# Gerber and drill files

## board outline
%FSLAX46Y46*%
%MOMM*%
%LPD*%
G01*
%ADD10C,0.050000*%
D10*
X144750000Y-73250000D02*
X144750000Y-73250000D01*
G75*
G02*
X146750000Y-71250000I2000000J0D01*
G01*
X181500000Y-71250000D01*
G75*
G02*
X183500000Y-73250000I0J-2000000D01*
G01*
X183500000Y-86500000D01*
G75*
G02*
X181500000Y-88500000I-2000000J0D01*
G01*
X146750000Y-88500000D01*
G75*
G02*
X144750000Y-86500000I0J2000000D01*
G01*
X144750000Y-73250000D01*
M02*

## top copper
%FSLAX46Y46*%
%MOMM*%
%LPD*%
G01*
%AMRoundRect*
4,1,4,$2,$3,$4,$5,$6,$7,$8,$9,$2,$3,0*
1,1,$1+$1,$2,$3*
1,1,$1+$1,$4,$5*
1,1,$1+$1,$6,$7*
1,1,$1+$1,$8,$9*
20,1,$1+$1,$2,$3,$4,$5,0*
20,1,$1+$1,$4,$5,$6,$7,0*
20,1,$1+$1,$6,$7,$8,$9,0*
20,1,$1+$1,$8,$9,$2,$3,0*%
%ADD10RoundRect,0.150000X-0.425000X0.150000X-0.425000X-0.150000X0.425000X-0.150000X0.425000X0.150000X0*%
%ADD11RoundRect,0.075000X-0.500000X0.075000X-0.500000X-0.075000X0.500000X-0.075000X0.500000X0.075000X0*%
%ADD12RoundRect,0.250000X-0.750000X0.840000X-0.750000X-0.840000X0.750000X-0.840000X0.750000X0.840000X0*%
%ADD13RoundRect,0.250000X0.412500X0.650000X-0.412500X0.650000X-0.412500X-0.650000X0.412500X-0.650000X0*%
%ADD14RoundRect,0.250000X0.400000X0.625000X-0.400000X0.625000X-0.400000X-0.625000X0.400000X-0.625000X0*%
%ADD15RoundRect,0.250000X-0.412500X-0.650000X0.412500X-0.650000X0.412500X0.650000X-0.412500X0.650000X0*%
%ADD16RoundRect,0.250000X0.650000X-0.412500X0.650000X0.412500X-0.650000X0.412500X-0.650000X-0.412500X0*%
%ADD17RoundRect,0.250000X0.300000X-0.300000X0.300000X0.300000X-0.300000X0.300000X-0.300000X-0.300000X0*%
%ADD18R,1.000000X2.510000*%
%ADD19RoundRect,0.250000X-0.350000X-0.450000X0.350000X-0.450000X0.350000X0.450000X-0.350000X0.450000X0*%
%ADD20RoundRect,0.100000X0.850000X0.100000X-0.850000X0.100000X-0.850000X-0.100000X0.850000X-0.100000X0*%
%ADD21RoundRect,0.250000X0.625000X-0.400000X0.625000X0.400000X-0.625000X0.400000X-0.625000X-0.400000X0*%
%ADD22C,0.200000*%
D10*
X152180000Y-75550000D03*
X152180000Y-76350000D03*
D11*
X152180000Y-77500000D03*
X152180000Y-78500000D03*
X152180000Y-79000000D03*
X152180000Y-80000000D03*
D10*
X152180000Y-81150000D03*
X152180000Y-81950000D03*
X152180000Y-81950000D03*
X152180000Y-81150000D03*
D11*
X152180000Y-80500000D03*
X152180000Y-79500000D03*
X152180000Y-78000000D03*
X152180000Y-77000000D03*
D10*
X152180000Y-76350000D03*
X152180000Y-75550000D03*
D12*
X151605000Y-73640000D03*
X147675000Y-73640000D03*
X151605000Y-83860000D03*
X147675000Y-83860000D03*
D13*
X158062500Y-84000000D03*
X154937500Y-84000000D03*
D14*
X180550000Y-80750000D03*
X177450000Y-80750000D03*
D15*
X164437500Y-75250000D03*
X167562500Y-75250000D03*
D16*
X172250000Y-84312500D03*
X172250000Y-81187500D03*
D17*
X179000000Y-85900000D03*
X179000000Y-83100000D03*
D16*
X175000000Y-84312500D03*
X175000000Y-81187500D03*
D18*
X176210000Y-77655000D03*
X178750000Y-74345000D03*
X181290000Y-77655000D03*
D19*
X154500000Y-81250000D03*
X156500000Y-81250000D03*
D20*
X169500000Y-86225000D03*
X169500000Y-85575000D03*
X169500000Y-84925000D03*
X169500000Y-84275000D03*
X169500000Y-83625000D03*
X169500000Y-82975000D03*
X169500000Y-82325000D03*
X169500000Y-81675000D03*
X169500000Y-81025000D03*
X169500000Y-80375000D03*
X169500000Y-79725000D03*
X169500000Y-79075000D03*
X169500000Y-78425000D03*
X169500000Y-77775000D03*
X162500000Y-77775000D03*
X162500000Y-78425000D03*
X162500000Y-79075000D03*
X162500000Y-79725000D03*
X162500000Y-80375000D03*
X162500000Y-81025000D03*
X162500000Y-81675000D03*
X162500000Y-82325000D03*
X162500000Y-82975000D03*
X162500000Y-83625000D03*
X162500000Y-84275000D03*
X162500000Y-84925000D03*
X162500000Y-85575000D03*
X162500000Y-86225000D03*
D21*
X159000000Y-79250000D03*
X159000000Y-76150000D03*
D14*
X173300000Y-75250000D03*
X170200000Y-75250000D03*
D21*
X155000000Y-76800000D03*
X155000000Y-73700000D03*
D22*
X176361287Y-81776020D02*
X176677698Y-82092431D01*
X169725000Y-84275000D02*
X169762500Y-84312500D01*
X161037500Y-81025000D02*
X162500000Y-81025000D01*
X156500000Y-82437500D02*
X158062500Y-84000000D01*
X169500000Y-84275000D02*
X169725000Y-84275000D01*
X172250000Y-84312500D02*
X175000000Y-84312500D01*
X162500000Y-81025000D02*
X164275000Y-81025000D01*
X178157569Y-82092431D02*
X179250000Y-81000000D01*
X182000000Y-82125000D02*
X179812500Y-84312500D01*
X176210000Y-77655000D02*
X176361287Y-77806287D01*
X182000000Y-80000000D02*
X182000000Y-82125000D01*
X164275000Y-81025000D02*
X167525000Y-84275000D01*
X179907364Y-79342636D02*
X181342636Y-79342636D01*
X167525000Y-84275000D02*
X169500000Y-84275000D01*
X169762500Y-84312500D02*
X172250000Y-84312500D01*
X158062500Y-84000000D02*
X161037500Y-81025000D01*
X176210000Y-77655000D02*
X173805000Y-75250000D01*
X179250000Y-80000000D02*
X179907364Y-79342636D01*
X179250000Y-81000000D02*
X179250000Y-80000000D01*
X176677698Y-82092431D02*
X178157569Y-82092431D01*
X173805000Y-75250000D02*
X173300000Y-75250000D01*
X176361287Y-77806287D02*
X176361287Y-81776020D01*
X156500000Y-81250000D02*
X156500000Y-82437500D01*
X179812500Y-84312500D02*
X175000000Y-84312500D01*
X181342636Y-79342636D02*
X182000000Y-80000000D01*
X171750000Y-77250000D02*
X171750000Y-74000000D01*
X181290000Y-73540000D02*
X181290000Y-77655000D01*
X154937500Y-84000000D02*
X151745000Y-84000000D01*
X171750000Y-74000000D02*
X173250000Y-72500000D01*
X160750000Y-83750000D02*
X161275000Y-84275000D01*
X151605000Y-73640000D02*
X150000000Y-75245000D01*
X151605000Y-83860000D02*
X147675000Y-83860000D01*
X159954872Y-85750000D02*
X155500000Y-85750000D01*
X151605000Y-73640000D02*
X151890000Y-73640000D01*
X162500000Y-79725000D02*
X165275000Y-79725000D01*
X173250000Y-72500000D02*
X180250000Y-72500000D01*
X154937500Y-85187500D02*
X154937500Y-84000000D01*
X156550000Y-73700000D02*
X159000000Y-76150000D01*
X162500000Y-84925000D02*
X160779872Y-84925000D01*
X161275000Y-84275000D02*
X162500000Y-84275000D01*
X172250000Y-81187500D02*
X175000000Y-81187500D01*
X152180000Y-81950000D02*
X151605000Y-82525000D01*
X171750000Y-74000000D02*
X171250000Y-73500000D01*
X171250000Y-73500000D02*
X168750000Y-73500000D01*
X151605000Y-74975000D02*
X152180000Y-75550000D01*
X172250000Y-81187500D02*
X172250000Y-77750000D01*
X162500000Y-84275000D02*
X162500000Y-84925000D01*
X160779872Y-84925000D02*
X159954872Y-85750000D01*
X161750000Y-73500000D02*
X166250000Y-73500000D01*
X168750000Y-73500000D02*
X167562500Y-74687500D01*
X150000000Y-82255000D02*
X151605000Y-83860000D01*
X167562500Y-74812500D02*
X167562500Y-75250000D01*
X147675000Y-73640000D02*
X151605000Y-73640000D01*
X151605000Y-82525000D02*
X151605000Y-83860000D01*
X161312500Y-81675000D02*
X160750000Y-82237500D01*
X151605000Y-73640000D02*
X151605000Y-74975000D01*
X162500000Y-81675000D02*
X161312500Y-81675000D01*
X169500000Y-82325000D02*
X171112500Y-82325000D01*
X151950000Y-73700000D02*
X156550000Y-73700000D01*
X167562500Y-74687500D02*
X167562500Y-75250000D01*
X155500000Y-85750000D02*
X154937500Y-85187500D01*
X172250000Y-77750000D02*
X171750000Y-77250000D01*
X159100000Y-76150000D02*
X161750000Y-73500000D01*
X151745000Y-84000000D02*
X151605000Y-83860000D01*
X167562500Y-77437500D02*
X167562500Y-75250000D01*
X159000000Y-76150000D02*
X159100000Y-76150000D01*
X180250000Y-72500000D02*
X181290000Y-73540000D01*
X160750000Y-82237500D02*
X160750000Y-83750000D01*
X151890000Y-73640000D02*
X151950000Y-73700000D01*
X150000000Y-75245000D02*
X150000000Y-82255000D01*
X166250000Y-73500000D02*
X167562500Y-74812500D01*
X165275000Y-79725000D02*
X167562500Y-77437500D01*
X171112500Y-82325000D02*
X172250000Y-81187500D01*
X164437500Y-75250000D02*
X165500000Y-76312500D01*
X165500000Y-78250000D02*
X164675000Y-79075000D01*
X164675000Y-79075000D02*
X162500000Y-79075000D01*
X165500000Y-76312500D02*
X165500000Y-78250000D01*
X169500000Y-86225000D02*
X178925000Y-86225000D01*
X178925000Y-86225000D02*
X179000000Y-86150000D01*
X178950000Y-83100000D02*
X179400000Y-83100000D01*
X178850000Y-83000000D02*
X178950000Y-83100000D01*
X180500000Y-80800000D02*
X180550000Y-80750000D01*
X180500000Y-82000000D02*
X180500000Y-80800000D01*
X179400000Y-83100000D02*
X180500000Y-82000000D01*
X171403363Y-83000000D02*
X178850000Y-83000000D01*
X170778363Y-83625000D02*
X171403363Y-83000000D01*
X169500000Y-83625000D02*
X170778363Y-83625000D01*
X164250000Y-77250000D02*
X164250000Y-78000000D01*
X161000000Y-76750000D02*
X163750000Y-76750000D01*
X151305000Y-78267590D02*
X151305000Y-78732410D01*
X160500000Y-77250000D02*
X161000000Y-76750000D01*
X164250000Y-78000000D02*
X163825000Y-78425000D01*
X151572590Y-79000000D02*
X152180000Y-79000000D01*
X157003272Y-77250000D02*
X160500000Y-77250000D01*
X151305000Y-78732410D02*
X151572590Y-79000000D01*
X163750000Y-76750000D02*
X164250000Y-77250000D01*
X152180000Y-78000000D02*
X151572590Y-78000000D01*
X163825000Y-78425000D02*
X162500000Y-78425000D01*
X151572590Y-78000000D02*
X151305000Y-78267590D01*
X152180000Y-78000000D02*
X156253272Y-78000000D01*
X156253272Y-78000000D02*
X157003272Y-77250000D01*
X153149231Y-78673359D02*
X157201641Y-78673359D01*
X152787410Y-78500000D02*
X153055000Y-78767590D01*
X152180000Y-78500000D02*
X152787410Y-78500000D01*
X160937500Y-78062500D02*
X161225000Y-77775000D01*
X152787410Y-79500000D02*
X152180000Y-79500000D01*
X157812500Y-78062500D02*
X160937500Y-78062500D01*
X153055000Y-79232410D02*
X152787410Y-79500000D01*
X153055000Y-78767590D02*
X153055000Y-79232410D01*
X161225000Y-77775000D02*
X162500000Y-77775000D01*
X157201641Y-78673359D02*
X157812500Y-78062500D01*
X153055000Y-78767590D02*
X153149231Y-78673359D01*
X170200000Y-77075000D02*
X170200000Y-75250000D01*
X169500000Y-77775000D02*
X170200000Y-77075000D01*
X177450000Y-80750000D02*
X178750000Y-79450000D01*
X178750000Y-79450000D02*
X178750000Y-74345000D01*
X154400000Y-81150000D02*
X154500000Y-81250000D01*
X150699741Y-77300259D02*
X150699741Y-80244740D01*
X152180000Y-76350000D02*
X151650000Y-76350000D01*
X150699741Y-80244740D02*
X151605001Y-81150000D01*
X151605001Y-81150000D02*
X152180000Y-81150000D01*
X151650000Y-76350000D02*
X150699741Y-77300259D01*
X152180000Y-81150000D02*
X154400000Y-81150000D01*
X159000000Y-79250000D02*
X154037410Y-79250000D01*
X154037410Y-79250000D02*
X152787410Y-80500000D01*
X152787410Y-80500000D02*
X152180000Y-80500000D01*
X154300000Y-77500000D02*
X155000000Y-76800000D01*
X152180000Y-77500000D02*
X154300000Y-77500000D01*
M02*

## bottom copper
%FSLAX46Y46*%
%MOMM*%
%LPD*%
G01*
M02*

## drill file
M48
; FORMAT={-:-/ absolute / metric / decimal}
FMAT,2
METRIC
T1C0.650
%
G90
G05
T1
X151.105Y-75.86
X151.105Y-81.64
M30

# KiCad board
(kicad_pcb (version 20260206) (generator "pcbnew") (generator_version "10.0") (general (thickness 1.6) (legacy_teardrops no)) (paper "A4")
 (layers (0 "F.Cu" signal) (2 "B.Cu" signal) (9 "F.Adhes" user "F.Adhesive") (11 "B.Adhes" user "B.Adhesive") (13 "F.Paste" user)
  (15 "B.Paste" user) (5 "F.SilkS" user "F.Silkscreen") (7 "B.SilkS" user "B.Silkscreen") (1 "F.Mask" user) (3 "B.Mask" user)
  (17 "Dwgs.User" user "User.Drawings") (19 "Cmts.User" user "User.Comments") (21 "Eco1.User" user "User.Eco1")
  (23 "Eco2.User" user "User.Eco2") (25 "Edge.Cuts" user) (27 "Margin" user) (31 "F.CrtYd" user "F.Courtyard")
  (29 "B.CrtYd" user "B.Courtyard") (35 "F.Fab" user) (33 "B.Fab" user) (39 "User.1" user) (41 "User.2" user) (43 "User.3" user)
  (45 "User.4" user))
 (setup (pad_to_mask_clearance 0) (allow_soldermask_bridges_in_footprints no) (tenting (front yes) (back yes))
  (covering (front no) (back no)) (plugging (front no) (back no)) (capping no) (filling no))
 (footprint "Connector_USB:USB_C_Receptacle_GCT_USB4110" (layer "F.Cu") (at 148.5 78.75 -90)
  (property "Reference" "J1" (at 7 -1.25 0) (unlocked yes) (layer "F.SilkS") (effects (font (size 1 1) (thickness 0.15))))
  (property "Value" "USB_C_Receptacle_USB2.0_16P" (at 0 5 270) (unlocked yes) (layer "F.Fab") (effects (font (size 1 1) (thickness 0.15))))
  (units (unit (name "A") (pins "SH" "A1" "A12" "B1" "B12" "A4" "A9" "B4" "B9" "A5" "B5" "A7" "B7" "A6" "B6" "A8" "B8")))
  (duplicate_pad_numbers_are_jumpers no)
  (pad "" np_thru_hole circle (at -2.89 -2.605 270) (size 0.65 0.65) (drill 0.65) (layers "*.Cu" "*.Mask"))
  (pad "" np_thru_hole circle (at 2.89 -2.605 270) (size 0.65 0.65) (drill 0.65) (layers "*.Cu" "*.Mask"))
  (pad "A1" smd roundrect (at -3.2 -3.68 270) (size 0.6 1.15) (layers "F.Cu" "F.Mask" "F.Paste") (roundrect_rratio 0.25) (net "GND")
   (thermal_bridge_angle 45))
  (pad "A4" smd roundrect (at -2.4 -3.68 270) (size 0.6 1.15) (layers "F.Cu" "F.Mask" "F.Paste") (roundrect_rratio 0.25)
   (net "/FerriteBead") (thermal_bridge_angle 45))
  (pad "A5" smd roundrect (at -1.25 -3.68 270) (size 0.3 1.15) (layers "F.Cu" "F.Mask" "F.Paste") (roundrect_rratio 0.25) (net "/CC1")
   (thermal_bridge_angle 45))
  (pad "A6" smd roundrect (at -0.25 -3.68 270) (size 0.3 1.15) (layers "F.Cu" "F.Mask" "F.Paste") (roundrect_rratio 0.25) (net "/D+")
   (thermal_bridge_angle 45))
  (pad "A7" smd roundrect (at 0.25 -3.68 270) (size 0.3 1.15) (layers "F.Cu" "F.Mask" "F.Paste") (roundrect_rratio 0.25) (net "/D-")
   (thermal_bridge_angle 45))
  (pad "A8" smd roundrect (at 1.25 -3.68 270) (size 0.3 1.15) (layers "F.Cu" "F.Mask" "F.Paste") (roundrect_rratio 0.25) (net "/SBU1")
   (thermal_bridge_angle 45))
  (pad "A9" smd roundrect (at 2.4 -3.68 270) (size 0.6 1.15) (layers "F.Cu" "F.Mask" "F.Paste") (roundrect_rratio 0.25) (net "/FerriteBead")
   (thermal_bridge_angle 45))
  (pad "A12" smd roundrect (at 3.2 -3.68 270) (size 0.6 1.15) (layers "F.Cu" "F.Mask" "F.Paste") (roundrect_rratio 0.25) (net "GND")
   (thermal_bridge_angle 45))
  (pad "B1" smd roundrect (at 3.2 -3.68 270) (size 0.6 1.15) (layers "F.Cu" "F.Mask" "F.Paste") (roundrect_rratio 0.25) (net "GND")
   (thermal_bridge_angle 45))
  (pad "B4" smd roundrect (at 2.4 -3.68 270) (size 0.6 1.15) (layers "F.Cu" "F.Mask" "F.Paste") (roundrect_rratio 0.25) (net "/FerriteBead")
   (thermal_bridge_angle 45))
  (pad "B5" smd roundrect (at 1.75 -3.68 270) (size 0.3 1.15) (layers "F.Cu" "F.Mask" "F.Paste") (roundrect_rratio 0.25) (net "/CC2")
   (thermal_bridge_angle 45))
  (pad "B6" smd roundrect (at 0.75 -3.68 270) (size 0.3 1.15) (layers "F.Cu" "F.Mask" "F.Paste") (roundrect_rratio 0.25) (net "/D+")
   (thermal_bridge_angle 45))
  (pad "B7" smd roundrect (at -0.75 -3.68 270) (size 0.3 1.15) (layers "F.Cu" "F.Mask" "F.Paste") (roundrect_rratio 0.25) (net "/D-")
   (thermal_bridge_angle 45))
  (pad "B8" smd roundrect (at -1.75 -3.68 270) (size 0.3 1.15) (layers "F.Cu" "F.Mask" "F.Paste") (roundrect_rratio 0.25) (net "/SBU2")
   (thermal_bridge_angle 45))
  (pad "B9" smd roundrect (at -2.4 -3.68 270) (size 0.6 1.15) (layers "F.Cu" "F.Mask" "F.Paste") (roundrect_rratio 0.25)
   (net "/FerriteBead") (thermal_bridge_angle 45))
  (pad "B12" smd roundrect (at -3.2 -3.68 270) (size 0.6 1.15) (layers "F.Cu" "F.Mask" "F.Paste") (roundrect_rratio 0.25) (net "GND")
   (thermal_bridge_angle 45))
  (pad "SH" smd roundrect (at -5.11 -3.105 270) (size 2.18 2) (layers "F.Cu" "F.Mask" "F.Paste") (roundrect_rratio 0.125) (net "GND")
   (thermal_bridge_angle 45))
  (pad "SH" smd roundrect (at -5.11 0.825 270) (size 2.18 2) (layers "F.Cu" "F.Mask" "F.Paste") (roundrect_rratio 0.125) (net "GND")
   (thermal_bridge_angle 45))
  (pad "SH" smd roundrect (at 5.11 -3.105 270) (size 2.18 2) (layers "F.Cu" "F.Mask" "F.Paste") (roundrect_rratio 0.125) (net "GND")
   (thermal_bridge_angle 45))
  (pad "SH" smd roundrect (at 5.11 0.825 270) (size 2.18 2) (layers "F.Cu" "F.Mask" "F.Paste") (roundrect_rratio 0.125) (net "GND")
   (thermal_bridge_angle 45)))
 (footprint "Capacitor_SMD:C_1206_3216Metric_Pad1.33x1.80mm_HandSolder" (layer "F.Cu") (at 156.5 84 180)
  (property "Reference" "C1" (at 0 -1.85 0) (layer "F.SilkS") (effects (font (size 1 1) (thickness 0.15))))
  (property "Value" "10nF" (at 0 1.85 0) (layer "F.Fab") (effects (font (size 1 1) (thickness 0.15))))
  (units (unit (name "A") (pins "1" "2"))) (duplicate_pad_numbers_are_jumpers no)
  (pad "1" smd roundrect (at -1.5625 0 180) (size 1.325 1.8) (layers "F.Cu" "F.Mask" "F.Paste") (roundrect_rratio 0.188679) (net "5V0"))
  (pad "2" smd roundrect (at 1.5625 0 180) (size 1.325 1.8) (layers "F.Cu" "F.Mask" "F.Paste") (roundrect_rratio 0.188679) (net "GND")))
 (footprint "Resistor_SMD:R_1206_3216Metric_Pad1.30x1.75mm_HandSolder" (layer "F.Cu") (at 179 80.75 180)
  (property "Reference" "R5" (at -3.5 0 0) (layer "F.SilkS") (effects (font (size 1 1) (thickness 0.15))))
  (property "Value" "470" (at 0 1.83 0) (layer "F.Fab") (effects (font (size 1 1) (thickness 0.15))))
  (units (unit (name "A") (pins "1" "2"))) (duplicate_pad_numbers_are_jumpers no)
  (pad "1" smd roundrect (at -1.55 0 180) (size 1.3 1.75) (layers "F.Cu" "F.Mask" "F.Paste") (roundrect_rratio 0.192308) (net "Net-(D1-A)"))
  (pad "2" smd roundrect (at 1.55 0 180) (size 1.3 1.75) (layers "F.Cu" "F.Mask" "F.Paste") (roundrect_rratio 0.192308)
   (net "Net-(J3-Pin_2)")))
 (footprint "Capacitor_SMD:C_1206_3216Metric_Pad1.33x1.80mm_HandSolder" (layer "F.Cu") (at 166 75.25)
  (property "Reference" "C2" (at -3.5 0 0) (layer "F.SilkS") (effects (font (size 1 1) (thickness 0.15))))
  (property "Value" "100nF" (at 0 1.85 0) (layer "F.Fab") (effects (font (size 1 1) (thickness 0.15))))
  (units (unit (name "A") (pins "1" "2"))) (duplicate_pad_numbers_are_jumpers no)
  (pad "1" smd roundrect (at -1.5625 0) (size 1.325 1.8) (layers "F.Cu" "F.Mask" "F.Paste") (roundrect_rratio 0.188679)
   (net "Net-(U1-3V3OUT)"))
  (pad "2" smd roundrect (at 1.5625 0) (size 1.325 1.8) (layers "F.Cu" "F.Mask" "F.Paste") (roundrect_rratio 0.188679) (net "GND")))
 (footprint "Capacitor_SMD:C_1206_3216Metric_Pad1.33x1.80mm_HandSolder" (layer "F.Cu") (at 172.25 82.75 90)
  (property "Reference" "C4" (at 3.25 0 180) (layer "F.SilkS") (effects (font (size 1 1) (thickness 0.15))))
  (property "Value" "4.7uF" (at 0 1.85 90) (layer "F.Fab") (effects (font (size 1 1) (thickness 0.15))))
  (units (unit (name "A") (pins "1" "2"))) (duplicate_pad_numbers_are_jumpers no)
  (pad "1" smd roundrect (at -1.5625 0 90) (size 1.325 1.8) (layers "F.Cu" "F.Mask" "F.Paste") (roundrect_rratio 0.188679) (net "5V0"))
  (pad "2" smd roundrect (at 1.5625 0 90) (size 1.325 1.8) (layers "F.Cu" "F.Mask" "F.Paste") (roundrect_rratio 0.188679) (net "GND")))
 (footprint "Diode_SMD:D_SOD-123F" (layer "F.Cu") (at 179 84.5 90)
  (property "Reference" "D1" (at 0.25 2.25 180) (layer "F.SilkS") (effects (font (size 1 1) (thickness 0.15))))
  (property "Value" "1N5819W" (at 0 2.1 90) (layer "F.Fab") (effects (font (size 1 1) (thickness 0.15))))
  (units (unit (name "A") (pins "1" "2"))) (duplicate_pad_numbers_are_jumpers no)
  (pad "1" smd roundrect (at -1.4 0 90) (size 1.1 1.1) (layers "F.Cu" "F.Mask" "F.Paste") (roundrect_rratio 0.2272727273) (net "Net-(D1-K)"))
  (pad "2" smd roundrect (at 1.4 0 90) (size 1.1 1.1) (layers "F.Cu" "F.Mask" "F.Paste") (roundrect_rratio 0.2272727273) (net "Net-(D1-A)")))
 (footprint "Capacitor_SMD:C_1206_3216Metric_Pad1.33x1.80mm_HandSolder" (layer "F.Cu") (at 175 82.75 90)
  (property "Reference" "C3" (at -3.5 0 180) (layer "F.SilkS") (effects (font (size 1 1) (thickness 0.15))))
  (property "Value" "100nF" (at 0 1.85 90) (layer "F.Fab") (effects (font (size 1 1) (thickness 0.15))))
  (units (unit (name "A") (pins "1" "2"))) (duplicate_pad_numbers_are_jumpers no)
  (pad "1" smd roundrect (at -1.5625 0 90) (size 1.325 1.8) (layers "F.Cu" "F.Mask" "F.Paste") (roundrect_rratio 0.188679) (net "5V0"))
  (pad "2" smd roundrect (at 1.5625 0 90) (size 1.325 1.8) (layers "F.Cu" "F.Mask" "F.Paste") (roundrect_rratio 0.188679) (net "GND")))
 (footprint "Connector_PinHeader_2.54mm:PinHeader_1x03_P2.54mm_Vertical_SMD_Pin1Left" (layer "F.Cu") (at 178.75 76 90)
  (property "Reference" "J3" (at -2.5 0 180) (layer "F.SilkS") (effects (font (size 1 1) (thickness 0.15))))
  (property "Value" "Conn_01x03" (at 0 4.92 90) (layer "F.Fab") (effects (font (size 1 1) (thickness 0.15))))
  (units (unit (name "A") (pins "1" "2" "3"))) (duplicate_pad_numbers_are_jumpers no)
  (pad "1" smd rect (at -1.655 -2.54 90) (size 2.51 1) (layers "F.Cu" "F.Mask" "F.Paste") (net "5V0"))
  (pad "2" smd rect (at 1.655 0 90) (size 2.51 1) (layers "F.Cu" "F.Mask" "F.Paste") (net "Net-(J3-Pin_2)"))
  (pad "3" smd rect (at -1.655 2.54 90) (size 2.51 1) (layers "F.Cu" "F.Mask" "F.Paste") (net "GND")))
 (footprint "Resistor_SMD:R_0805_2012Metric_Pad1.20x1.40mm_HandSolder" (layer "F.Cu") (at 155.5 81.25)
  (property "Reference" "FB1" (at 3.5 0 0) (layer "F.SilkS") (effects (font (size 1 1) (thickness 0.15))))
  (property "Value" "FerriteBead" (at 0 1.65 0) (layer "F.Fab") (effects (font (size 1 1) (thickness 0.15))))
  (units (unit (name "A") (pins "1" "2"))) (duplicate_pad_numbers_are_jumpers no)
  (pad "1" smd roundrect (at -1 0) (size 1.2 1.4) (layers "F.Cu" "F.Mask" "F.Paste") (roundrect_rratio 0.208333) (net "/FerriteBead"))
  (pad "2" smd roundrect (at 1 0) (size 1.2 1.4) (layers "F.Cu" "F.Mask" "F.Paste") (roundrect_rratio 0.208333) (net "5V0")))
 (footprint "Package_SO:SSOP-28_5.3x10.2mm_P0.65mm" (layer "F.Cu") (at 166 82 180)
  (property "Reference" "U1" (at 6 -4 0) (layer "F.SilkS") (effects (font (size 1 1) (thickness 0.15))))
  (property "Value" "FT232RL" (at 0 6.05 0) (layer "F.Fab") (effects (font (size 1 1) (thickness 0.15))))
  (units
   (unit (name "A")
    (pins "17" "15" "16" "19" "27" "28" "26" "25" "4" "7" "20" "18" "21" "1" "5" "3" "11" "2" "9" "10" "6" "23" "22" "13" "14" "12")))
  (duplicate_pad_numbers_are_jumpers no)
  (pad "1" smd roundrect (at -3.5 -4.225 180) (size 1.9 0.4) (layers "F.Cu" "F.Mask" "F.Paste") (roundrect_rratio 0.25) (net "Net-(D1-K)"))
  (pad "2" smd roundrect (at -3.5 -3.575 180) (size 1.9 0.4) (layers "F.Cu" "F.Mask" "F.Paste") (roundrect_rratio 0.25)
   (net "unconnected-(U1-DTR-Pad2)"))
  (pad "3" smd roundrect (at -3.5 -2.925 180) (size 1.9 0.4) (layers "F.Cu" "F.Mask" "F.Paste") (roundrect_rratio 0.25)
   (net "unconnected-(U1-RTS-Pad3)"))
  (pad "4" smd roundrect (at -3.5 -2.275 180) (size 1.9 0.4) (layers "F.Cu" "F.Mask" "F.Paste") (roundrect_rratio 0.25) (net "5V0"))
  (pad "5" smd roundrect (at -3.5 -1.625 180) (size 1.9 0.4) (layers "F.Cu" "F.Mask" "F.Paste") (roundrect_rratio 0.25) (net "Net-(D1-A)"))
  (pad "6" smd roundrect (at -3.5 -0.975 180) (size 1.9 0.4) (layers "F.Cu" "F.Mask" "F.Paste") (roundrect_rratio 0.25)
   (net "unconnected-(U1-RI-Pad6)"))
  (pad "7" smd roundrect (at -3.5 -0.325 180) (size 1.9 0.4) (layers "F.Cu" "F.Mask" "F.Paste") (roundrect_rratio 0.25) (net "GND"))
  (pad "8" smd roundrect (at -3.5 0.325 180) (size 1.9 0.4) (layers "F.Cu" "F.Mask" "F.Paste") (roundrect_rratio 0.25))
  (pad "9" smd roundrect (at -3.5 0.975 180) (size 1.9 0.4) (layers "F.Cu" "F.Mask" "F.Paste") (roundrect_rratio 0.25)
   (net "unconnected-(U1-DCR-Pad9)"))
  (pad "10" smd roundrect (at -3.5 1.625 180) (size 1.9 0.4) (layers "F.Cu" "F.Mask" "F.Paste") (roundrect_rratio 0.25)
   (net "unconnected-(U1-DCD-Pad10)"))
  (pad "11" smd roundrect (at -3.5 2.275 180) (size 1.9 0.4) (layers "F.Cu" "F.Mask" "F.Paste") (roundrect_rratio 0.25)
   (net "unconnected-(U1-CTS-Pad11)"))
  (pad "12" smd roundrect (at -3.5 2.925 180) (size 1.9 0.4) (layers "F.Cu" "F.Mask" "F.Paste") (roundrect_rratio 0.25)
   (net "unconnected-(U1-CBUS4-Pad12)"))
  (pad "13" smd roundrect (at -3.5 3.575 180) (size 1.9 0.4) (layers "F.Cu" "F.Mask" "F.Paste") (roundrect_rratio 0.25)
   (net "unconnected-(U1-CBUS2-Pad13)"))
  (pad "14" smd roundrect (at -3.5 4.225 180) (size 1.9 0.4) (layers "F.Cu" "F.Mask" "F.Paste") (roundrect_rratio 0.25)
   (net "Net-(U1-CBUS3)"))
  (pad "15" smd roundrect (at 3.5 4.225 180) (size 1.9 0.4) (layers "F.Cu" "F.Mask" "F.Paste") (roundrect_rratio 0.25) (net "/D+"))
  (pad "16" smd roundrect (at 3.5 3.575 180) (size 1.9 0.4) (layers "F.Cu" "F.Mask" "F.Paste") (roundrect_rratio 0.25) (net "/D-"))
  (pad "17" smd roundrect (at 3.5 2.925 180) (size 1.9 0.4) (layers "F.Cu" "F.Mask" "F.Paste") (roundrect_rratio 0.25)
   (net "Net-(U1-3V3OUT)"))
  (pad "18" smd roundrect (at 3.5 2.275 180) (size 1.9 0.4) (layers "F.Cu" "F.Mask" "F.Paste") (roundrect_rratio 0.25) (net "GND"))
  (pad "19" smd roundrect (at 3.5 1.625 180) (size 1.9 0.4) (layers "F.Cu" "F.Mask" "F.Paste") (roundrect_rratio 0.25)
   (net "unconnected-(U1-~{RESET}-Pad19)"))
  (pad "20" smd roundrect (at 3.5 0.975 180) (size 1.9 0.4) (layers "F.Cu" "F.Mask" "F.Paste") (roundrect_rratio 0.25) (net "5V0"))
  (pad "21" smd roundrect (at 3.5 0.325 180) (size 1.9 0.4) (layers "F.Cu" "F.Mask" "F.Paste") (roundrect_rratio 0.25) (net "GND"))
  (pad "22" smd roundrect (at 3.5 -0.325 180) (size 1.9 0.4) (layers "F.Cu" "F.Mask" "F.Paste") (roundrect_rratio 0.25)
   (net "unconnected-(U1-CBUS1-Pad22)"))
  (pad "23" smd roundrect (at 3.5 -0.975 180) (size 1.9 0.4) (layers "F.Cu" "F.Mask" "F.Paste") (roundrect_rratio 0.25)
   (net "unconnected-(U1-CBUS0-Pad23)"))
  (pad "24" smd roundrect (at 3.5 -1.625 180) (size 1.9 0.4) (layers "F.Cu" "F.Mask" "F.Paste") (roundrect_rratio 0.25))
  (pad "25" smd roundrect (at 3.5 -2.275 180) (size 1.9 0.4) (layers "F.Cu" "F.Mask" "F.Paste") (roundrect_rratio 0.25) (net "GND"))
  (pad "26" smd roundrect (at 3.5 -2.925 180) (size 1.9 0.4) (layers "F.Cu" "F.Mask" "F.Paste") (roundrect_rratio 0.25) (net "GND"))
  (pad "27" smd roundrect (at 3.5 -3.575 180) (size 1.9 0.4) (layers "F.Cu" "F.Mask" "F.Paste") (roundrect_rratio 0.25)
   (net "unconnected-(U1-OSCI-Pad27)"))
  (pad "28" smd roundrect (at 3.5 -4.225 180) (size 1.9 0.4) (layers "F.Cu" "F.Mask" "F.Paste") (roundrect_rratio 0.25)
   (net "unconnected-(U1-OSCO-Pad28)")))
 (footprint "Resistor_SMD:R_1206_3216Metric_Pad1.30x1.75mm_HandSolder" (layer "F.Cu") (at 159 77.7 90)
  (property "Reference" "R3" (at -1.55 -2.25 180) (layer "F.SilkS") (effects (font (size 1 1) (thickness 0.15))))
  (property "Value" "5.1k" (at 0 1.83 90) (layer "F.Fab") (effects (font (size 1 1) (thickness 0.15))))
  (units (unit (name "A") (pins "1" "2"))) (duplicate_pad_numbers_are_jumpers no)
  (pad "1" smd roundrect (at -1.55 0 90) (size 1.3 1.75) (layers "F.Cu" "F.Mask" "F.Paste") (roundrect_rratio 0.192308) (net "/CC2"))
  (pad "2" smd roundrect (at 1.55 0 90) (size 1.3 1.75) (layers "F.Cu" "F.Mask" "F.Paste") (roundrect_rratio 0.192308) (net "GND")))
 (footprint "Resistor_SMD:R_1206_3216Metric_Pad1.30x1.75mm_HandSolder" (layer "F.Cu") (at 171.75 75.25 180)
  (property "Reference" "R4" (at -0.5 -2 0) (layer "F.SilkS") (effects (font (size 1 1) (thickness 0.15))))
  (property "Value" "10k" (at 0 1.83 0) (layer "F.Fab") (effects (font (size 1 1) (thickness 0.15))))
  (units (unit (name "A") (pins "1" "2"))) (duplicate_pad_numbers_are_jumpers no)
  (pad "1" smd roundrect (at -1.55 0 180) (size 1.3 1.75) (layers "F.Cu" "F.Mask" "F.Paste") (roundrect_rratio 0.192308) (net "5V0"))
  (pad "2" smd roundrect (at 1.55 0 180) (size 1.3 1.75) (layers "F.Cu" "F.Mask" "F.Paste") (roundrect_rratio 0.192308)
   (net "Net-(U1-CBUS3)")))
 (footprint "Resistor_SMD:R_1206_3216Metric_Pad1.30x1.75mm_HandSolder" (layer "F.Cu") (at 155 75.25 90)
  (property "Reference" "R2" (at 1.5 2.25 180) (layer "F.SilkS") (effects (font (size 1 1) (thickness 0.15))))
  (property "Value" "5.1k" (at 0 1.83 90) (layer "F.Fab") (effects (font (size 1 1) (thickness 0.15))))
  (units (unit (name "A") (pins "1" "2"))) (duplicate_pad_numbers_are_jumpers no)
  (pad "1" smd roundrect (at -1.55 0 90) (size 1.3 1.75) (layers "F.Cu" "F.Mask" "F.Paste") (roundrect_rratio 0.192308) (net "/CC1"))
  (pad "2" smd roundrect (at 1.55 0 90) (size 1.3 1.75) (layers "F.Cu" "F.Mask" "F.Paste") (roundrect_rratio 0.192308) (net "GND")))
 (gr_rect (start 144.75 71.25) (end 183.5 88.5) (radius 2) (stroke (width 0.05) (type solid)) (fill no) (layer "Edge.Cuts"))
 (segment (start 176.361287 81.77602) (end 176.677698 82.092431) (width 0.2) (layer "F.Cu") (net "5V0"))
 (segment (start 169.725 84.275) (end 169.7625 84.3125) (width 0.2) (layer "F.Cu") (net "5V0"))
 (segment (start 161.0375 81.025) (end 162.5 81.025) (width 0.2) (layer "F.Cu") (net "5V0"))
 (segment (start 156.5 82.4375) (end 158.0625 84) (width 0.2) (layer "F.Cu") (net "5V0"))
 (segment (start 169.5 84.275) (end 169.725 84.275) (width 0.2) (layer "F.Cu") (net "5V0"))
 (segment (start 172.25 84.3125) (end 175 84.3125) (width 0.2) (layer "F.Cu") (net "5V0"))
 (segment (start 162.5 81.025) (end 164.275 81.025) (width 0.2) (layer "F.Cu") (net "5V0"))
 (segment (start 178.157569 82.092431) (end 179.25 81) (width 0.2) (layer "F.Cu") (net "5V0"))
 (segment (start 182 82.125) (end 179.8125 84.3125) (width 0.2) (layer "F.Cu") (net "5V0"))
 (segment (start 176.21 77.655) (end 176.361287 77.806287) (width 0.2) (layer "F.Cu") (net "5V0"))
 (segment (start 182 80) (end 182 82.125) (width 0.2) (layer "F.Cu") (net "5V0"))
 (segment (start 164.275 81.025) (end 167.525 84.275) (width 0.2) (layer "F.Cu") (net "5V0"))
 (segment (start 179.907364 79.342636) (end 181.342636 79.342636) (width 0.2) (layer "F.Cu") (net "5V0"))
 (segment (start 167.525 84.275) (end 169.5 84.275) (width 0.2) (layer "F.Cu") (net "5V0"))
 (segment (start 169.7625 84.3125) (end 172.25 84.3125) (width 0.2) (layer "F.Cu") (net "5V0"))
 (segment (start 158.0625 84) (end 161.0375 81.025) (width 0.2) (layer "F.Cu") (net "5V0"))
 (segment (start 176.21 77.655) (end 173.805 75.25) (width 0.2) (layer "F.Cu") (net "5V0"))
 (segment (start 179.25 80) (end 179.907364 79.342636) (width 0.2) (layer "F.Cu") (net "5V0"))
 (segment (start 179.25 81) (end 179.25 80) (width 0.2) (layer "F.Cu") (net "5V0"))
 (segment (start 176.677698 82.092431) (end 178.157569 82.092431) (width 0.2) (layer "F.Cu") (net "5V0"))
 (segment (start 173.805 75.25) (end 173.3 75.25) (width 0.2) (layer "F.Cu") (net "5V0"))
 (segment (start 176.361287 77.806287) (end 176.361287 81.77602) (width 0.2) (layer "F.Cu") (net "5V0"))
 (segment (start 156.5 81.25) (end 156.5 82.4375) (width 0.2) (layer "F.Cu") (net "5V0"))
 (segment (start 179.8125 84.3125) (end 175 84.3125) (width 0.2) (layer "F.Cu") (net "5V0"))
 (segment (start 181.342636 79.342636) (end 182 80) (width 0.2) (layer "F.Cu") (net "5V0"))
 (segment (start 171.75 77.25) (end 171.75 74) (width 0.2) (layer "F.Cu") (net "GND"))
 (segment (start 181.29 73.54) (end 181.29 77.655) (width 0.2) (layer "F.Cu") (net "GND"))
 (segment (start 154.9375 84) (end 151.745 84) (width 0.2) (layer "F.Cu") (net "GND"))
 (segment (start 171.75 74) (end 173.25 72.5) (width 0.2) (layer "F.Cu") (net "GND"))
 (segment (start 160.75 83.75) (end 161.275 84.275) (width 0.2) (layer "F.Cu") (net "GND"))
 (segment (start 151.605 73.64) (end 150 75.245) (width 0.2) (layer "F.Cu") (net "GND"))
 (segment (start 151.605 83.86) (end 147.675 83.86) (width 0.2) (layer "F.Cu") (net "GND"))
 (segment (start 159.954872 85.75) (end 155.5 85.75) (width 0.2) (layer "F.Cu") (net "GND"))
 (segment (start 151.605 73.64) (end 151.89 73.64) (width 0.2) (layer "F.Cu") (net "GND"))
 (segment (start 162.5 79.725) (end 165.275 79.725) (width 0.2) (layer "F.Cu") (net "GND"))
 (segment (start 173.25 72.5) (end 180.25 72.5) (width 0.2) (layer "F.Cu") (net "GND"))
 (segment (start 154.9375 85.1875) (end 154.9375 84) (width 0.2) (layer "F.Cu") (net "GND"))
 (segment (start 156.55 73.7) (end 159 76.15) (width 0.2) (layer "F.Cu") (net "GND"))
 (segment (start 162.5 84.925) (end 160.779872 84.925) (width 0.2) (layer "F.Cu") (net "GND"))
 (segment (start 161.275 84.275) (end 162.5 84.275) (width 0.2) (layer "F.Cu") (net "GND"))
 (segment (start 172.25 81.1875) (end 175 81.1875) (width 0.2) (layer "F.Cu") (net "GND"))
 (segment (start 152.18 81.95) (end 151.605 82.525) (width 0.2) (layer "F.Cu") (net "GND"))
 (segment (start 171.75 74) (end 171.25 73.5) (width 0.2) (layer "F.Cu") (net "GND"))
 (segment (start 171.25 73.5) (end 168.75 73.5) (width 0.2) (layer "F.Cu") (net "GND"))
 (segment (start 151.605 74.975) (end 152.18 75.55) (width 0.2) (layer "F.Cu") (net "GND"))
 (segment (start 172.25 81.1875) (end 172.25 77.75) (width 0.2) (layer "F.Cu") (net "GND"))
 (segment (start 162.5 84.275) (end 162.5 84.925) (width 0.2) (layer "F.Cu") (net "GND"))
 (segment (start 160.779872 84.925) (end 159.954872 85.75) (width 0.2) (layer "F.Cu") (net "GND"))
 (segment (start 161.75 73.5) (end 166.25 73.5) (width 0.2) (layer "F.Cu") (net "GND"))
 (segment (start 168.75 73.5) (end 167.5625 74.6875) (width 0.2) (layer "F.Cu") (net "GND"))
 (segment (start 150 82.255) (end 151.605 83.86) (width 0.2) (layer "F.Cu") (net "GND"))
 (segment (start 167.5625 74.8125) (end 167.5625 75.25) (width 0.2) (layer "F.Cu") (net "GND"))
 (segment (start 147.675 73.64) (end 151.605 73.64) (width 0.2) (layer "F.Cu") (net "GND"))
 (segment (start 151.605 82.525) (end 151.605 83.86) (width 0.2) (layer "F.Cu") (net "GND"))
 (segment (start 161.3125 81.675) (end 160.75 82.2375) (width 0.2) (layer "F.Cu") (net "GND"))
 (segment (start 151.605 73.64) (end 151.605 74.975) (width 0.2) (layer "F.Cu") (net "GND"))
 (segment (start 162.5 81.675) (end 161.3125 81.675) (width 0.2) (layer "F.Cu") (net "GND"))
 (segment (start 169.5 82.325) (end 171.1125 82.325) (width 0.2) (layer "F.Cu") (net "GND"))
 (segment (start 151.95 73.7) (end 156.55 73.7) (width 0.2) (layer "F.Cu") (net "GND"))
 (segment (start 167.5625 74.6875) (end 167.5625 75.25) (width 0.2) (layer "F.Cu") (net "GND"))
 (segment (start 155.5 85.75) (end 154.9375 85.1875) (width 0.2) (layer "F.Cu") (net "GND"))
 (segment (start 172.25 77.75) (end 171.75 77.25) (width 0.2) (layer "F.Cu") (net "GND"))
 (segment (start 159.1 76.15) (end 161.75 73.5) (width 0.2) (layer "F.Cu") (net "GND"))
 (segment (start 151.745 84) (end 151.605 83.86) (width 0.2) (layer "F.Cu") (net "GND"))
 (segment (start 167.5625 77.4375) (end 167.5625 75.25) (width 0.2) (layer "F.Cu") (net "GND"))
 (segment (start 159 76.15) (end 159.1 76.15) (width 0.2) (layer "F.Cu") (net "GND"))
 (segment (start 180.25 72.5) (end 181.29 73.54) (width 0.2) (layer "F.Cu") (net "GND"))
 (segment (start 160.75 82.2375) (end 160.75 83.75) (width 0.2) (layer "F.Cu") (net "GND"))
 (segment (start 151.89 73.64) (end 151.95 73.7) (width 0.2) (layer "F.Cu") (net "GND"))
 (segment (start 150 75.245) (end 150 82.255) (width 0.2) (layer "F.Cu") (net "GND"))
 (segment (start 166.25 73.5) (end 167.5625 74.8125) (width 0.2) (layer "F.Cu") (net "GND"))
 (segment (start 165.275 79.725) (end 167.5625 77.4375) (width 0.2) (layer "F.Cu") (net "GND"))
 (segment (start 171.1125 82.325) (end 172.25 81.1875) (width 0.2) (layer "F.Cu") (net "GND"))
 (segment (start 164.4375 75.25) (end 165.5 76.3125) (width 0.2) (layer "F.Cu") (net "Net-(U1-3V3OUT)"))
 (segment (start 165.5 78.25) (end 164.675 79.075) (width 0.2) (layer "F.Cu") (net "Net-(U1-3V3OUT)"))
 (segment (start 164.675 79.075) (end 162.5 79.075) (width 0.2) (layer "F.Cu") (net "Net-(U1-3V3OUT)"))
 (segment (start 165.5 76.3125) (end 165.5 78.25) (width 0.2) (layer "F.Cu") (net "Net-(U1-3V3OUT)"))
 (segment (start 169.5 86.225) (end 178.925 86.225) (width 0.2) (layer "F.Cu") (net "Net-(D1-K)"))
 (segment (start 178.925 86.225) (end 179 86.15) (width 0.2) (layer "F.Cu") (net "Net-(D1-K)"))
 (segment (start 178.95 83.1) (end 179.4 83.1) (width 0.2) (layer "F.Cu") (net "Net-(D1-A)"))
 (segment (start 178.85 83) (end 178.95 83.1) (width 0.2) (layer "F.Cu") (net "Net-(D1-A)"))
 (segment (start 180.5 80.8) (end 180.55 80.75) (width 0.2) (layer "F.Cu") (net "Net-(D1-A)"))
 (segment (start 180.5 82) (end 180.5 80.8) (width 0.2) (layer "F.Cu") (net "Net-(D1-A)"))
 (segment (start 179.4 83.1) (end 180.5 82) (width 0.2) (layer "F.Cu") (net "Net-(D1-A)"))
 (segment (start 171.403363 83) (end 178.85 83) (width 0.2) (layer "F.Cu") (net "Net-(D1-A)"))
 (segment (start 170.778363 83.625) (end 171.403363 83) (width 0.2) (layer "F.Cu") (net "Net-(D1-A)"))
 (segment (start 169.5 83.625) (end 170.778363 83.625) (width 0.2) (layer "F.Cu") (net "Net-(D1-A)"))
 (segment (start 164.25 77.25) (end 164.25 78) (width 0.2) (layer "F.Cu") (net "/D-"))
 (segment (start 161 76.75) (end 163.75 76.75) (width 0.2) (layer "F.Cu") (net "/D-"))
 (segment (start 151.305 78.26759) (end 151.305 78.73241) (width 0.2) (layer "F.Cu") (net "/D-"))
 (segment (start 160.5 77.25) (end 161 76.75) (width 0.2) (layer "F.Cu") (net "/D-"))
 (segment (start 164.25 78) (end 163.825 78.425) (width 0.2) (layer "F.Cu") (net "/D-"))
 (segment (start 151.57259 79) (end 152.18 79) (width 0.2) (layer "F.Cu") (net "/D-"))
 (segment (start 157.003272 77.25) (end 160.5 77.25) (width 0.2) (layer "F.Cu") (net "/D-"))
 (segment (start 151.305 78.73241) (end 151.57259 79) (width 0.2) (layer "F.Cu") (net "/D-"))
 (segment (start 163.75 76.75) (end 164.25 77.25) (width 0.2) (layer "F.Cu") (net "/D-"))
 (segment (start 152.18 78) (end 151.57259 78) (width 0.2) (layer "F.Cu") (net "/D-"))
 (segment (start 163.825 78.425) (end 162.5 78.425) (width 0.2) (layer "F.Cu") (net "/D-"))
 (segment (start 151.57259 78) (end 151.305 78.26759) (width 0.2) (layer "F.Cu") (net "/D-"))
 (segment (start 152.18 78) (end 156.253272 78) (width 0.2) (layer "F.Cu") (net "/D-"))
 (segment (start 156.253272 78) (end 157.003272 77.25) (width 0.2) (layer "F.Cu") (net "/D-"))
 (segment (start 153.149231 78.673359) (end 157.201641 78.673359) (width 0.2) (layer "F.Cu") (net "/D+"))
 (segment (start 152.78741 78.5) (end 153.055 78.76759) (width 0.2) (layer "F.Cu") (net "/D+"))
 (segment (start 152.18 78.5) (end 152.78741 78.5) (width 0.2) (layer "F.Cu") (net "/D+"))
 (segment (start 160.9375 78.0625) (end 161.225 77.775) (width 0.2) (layer "F.Cu") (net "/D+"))
 (segment (start 152.78741 79.5) (end 152.18 79.5) (width 0.2) (layer "F.Cu") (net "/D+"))
 (segment (start 157.8125 78.0625) (end 160.9375 78.0625) (width 0.2) (layer "F.Cu") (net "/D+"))
 (segment (start 153.055 79.23241) (end 152.78741 79.5) (width 0.2) (layer "F.Cu") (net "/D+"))
 (segment (start 153.055 78.76759) (end 153.055 79.23241) (width 0.2) (layer "F.Cu") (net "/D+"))
 (segment (start 161.225 77.775) (end 162.5 77.775) (width 0.2) (layer "F.Cu") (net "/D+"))
 (segment (start 157.201641 78.673359) (end 157.8125 78.0625) (width 0.2) (layer "F.Cu") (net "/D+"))
 (segment (start 153.055 78.76759) (end 153.149231 78.673359) (width 0.2) (layer "F.Cu") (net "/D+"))
 (segment (start 170.2 77.075) (end 170.2 75.25) (width 0.2) (layer "F.Cu") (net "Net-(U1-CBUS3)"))
 (segment (start 169.5 77.775) (end 170.2 77.075) (width 0.2) (layer "F.Cu") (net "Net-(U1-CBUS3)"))
 (segment (start 177.45 80.75) (end 178.75 79.45) (width 0.2) (layer "F.Cu") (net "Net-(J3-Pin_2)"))
 (segment (start 178.75 79.45) (end 178.75 74.345) (width 0.2) (layer "F.Cu") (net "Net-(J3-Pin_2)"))
 (segment (start 154.4 81.15) (end 154.5 81.25) (width 0.2) (layer "F.Cu") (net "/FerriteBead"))
 (segment (start 150.699741 77.300259) (end 150.699741 80.24474) (width 0.2) (layer "F.Cu") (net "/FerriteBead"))
 (segment (start 152.18 76.35) (end 151.65 76.35) (width 0.2) (layer "F.Cu") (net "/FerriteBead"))
 (segment (start 150.699741 80.24474) (end 151.605001 81.15) (width 0.2) (layer "F.Cu") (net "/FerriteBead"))
 (segment (start 151.605001 81.15) (end 152.18 81.15) (width 0.2) (layer "F.Cu") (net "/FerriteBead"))
 (segment (start 151.65 76.35) (end 150.699741 77.300259) (width 0.2) (layer "F.Cu") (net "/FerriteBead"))
 (segment (start 152.18 81.15) (end 154.4 81.15) (width 0.2) (layer "F.Cu") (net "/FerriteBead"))
 (segment (start 159 79.25) (end 154.03741 79.25) (width 0.2) (layer "F.Cu") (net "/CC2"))
 (segment (start 154.03741 79.25) (end 152.78741 80.5) (width 0.2) (layer "F.Cu") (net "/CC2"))
 (segment (start 152.78741 80.5) (end 152.18 80.5) (width 0.2) (layer "F.Cu") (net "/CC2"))
 (segment (start 154.3 77.5) (end 155 76.8) (width 0.2) (layer "F.Cu") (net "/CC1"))
 (segment (start 152.18 77.5) (end 154.3 77.5) (width 0.2) (layer "F.Cu") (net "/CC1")))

